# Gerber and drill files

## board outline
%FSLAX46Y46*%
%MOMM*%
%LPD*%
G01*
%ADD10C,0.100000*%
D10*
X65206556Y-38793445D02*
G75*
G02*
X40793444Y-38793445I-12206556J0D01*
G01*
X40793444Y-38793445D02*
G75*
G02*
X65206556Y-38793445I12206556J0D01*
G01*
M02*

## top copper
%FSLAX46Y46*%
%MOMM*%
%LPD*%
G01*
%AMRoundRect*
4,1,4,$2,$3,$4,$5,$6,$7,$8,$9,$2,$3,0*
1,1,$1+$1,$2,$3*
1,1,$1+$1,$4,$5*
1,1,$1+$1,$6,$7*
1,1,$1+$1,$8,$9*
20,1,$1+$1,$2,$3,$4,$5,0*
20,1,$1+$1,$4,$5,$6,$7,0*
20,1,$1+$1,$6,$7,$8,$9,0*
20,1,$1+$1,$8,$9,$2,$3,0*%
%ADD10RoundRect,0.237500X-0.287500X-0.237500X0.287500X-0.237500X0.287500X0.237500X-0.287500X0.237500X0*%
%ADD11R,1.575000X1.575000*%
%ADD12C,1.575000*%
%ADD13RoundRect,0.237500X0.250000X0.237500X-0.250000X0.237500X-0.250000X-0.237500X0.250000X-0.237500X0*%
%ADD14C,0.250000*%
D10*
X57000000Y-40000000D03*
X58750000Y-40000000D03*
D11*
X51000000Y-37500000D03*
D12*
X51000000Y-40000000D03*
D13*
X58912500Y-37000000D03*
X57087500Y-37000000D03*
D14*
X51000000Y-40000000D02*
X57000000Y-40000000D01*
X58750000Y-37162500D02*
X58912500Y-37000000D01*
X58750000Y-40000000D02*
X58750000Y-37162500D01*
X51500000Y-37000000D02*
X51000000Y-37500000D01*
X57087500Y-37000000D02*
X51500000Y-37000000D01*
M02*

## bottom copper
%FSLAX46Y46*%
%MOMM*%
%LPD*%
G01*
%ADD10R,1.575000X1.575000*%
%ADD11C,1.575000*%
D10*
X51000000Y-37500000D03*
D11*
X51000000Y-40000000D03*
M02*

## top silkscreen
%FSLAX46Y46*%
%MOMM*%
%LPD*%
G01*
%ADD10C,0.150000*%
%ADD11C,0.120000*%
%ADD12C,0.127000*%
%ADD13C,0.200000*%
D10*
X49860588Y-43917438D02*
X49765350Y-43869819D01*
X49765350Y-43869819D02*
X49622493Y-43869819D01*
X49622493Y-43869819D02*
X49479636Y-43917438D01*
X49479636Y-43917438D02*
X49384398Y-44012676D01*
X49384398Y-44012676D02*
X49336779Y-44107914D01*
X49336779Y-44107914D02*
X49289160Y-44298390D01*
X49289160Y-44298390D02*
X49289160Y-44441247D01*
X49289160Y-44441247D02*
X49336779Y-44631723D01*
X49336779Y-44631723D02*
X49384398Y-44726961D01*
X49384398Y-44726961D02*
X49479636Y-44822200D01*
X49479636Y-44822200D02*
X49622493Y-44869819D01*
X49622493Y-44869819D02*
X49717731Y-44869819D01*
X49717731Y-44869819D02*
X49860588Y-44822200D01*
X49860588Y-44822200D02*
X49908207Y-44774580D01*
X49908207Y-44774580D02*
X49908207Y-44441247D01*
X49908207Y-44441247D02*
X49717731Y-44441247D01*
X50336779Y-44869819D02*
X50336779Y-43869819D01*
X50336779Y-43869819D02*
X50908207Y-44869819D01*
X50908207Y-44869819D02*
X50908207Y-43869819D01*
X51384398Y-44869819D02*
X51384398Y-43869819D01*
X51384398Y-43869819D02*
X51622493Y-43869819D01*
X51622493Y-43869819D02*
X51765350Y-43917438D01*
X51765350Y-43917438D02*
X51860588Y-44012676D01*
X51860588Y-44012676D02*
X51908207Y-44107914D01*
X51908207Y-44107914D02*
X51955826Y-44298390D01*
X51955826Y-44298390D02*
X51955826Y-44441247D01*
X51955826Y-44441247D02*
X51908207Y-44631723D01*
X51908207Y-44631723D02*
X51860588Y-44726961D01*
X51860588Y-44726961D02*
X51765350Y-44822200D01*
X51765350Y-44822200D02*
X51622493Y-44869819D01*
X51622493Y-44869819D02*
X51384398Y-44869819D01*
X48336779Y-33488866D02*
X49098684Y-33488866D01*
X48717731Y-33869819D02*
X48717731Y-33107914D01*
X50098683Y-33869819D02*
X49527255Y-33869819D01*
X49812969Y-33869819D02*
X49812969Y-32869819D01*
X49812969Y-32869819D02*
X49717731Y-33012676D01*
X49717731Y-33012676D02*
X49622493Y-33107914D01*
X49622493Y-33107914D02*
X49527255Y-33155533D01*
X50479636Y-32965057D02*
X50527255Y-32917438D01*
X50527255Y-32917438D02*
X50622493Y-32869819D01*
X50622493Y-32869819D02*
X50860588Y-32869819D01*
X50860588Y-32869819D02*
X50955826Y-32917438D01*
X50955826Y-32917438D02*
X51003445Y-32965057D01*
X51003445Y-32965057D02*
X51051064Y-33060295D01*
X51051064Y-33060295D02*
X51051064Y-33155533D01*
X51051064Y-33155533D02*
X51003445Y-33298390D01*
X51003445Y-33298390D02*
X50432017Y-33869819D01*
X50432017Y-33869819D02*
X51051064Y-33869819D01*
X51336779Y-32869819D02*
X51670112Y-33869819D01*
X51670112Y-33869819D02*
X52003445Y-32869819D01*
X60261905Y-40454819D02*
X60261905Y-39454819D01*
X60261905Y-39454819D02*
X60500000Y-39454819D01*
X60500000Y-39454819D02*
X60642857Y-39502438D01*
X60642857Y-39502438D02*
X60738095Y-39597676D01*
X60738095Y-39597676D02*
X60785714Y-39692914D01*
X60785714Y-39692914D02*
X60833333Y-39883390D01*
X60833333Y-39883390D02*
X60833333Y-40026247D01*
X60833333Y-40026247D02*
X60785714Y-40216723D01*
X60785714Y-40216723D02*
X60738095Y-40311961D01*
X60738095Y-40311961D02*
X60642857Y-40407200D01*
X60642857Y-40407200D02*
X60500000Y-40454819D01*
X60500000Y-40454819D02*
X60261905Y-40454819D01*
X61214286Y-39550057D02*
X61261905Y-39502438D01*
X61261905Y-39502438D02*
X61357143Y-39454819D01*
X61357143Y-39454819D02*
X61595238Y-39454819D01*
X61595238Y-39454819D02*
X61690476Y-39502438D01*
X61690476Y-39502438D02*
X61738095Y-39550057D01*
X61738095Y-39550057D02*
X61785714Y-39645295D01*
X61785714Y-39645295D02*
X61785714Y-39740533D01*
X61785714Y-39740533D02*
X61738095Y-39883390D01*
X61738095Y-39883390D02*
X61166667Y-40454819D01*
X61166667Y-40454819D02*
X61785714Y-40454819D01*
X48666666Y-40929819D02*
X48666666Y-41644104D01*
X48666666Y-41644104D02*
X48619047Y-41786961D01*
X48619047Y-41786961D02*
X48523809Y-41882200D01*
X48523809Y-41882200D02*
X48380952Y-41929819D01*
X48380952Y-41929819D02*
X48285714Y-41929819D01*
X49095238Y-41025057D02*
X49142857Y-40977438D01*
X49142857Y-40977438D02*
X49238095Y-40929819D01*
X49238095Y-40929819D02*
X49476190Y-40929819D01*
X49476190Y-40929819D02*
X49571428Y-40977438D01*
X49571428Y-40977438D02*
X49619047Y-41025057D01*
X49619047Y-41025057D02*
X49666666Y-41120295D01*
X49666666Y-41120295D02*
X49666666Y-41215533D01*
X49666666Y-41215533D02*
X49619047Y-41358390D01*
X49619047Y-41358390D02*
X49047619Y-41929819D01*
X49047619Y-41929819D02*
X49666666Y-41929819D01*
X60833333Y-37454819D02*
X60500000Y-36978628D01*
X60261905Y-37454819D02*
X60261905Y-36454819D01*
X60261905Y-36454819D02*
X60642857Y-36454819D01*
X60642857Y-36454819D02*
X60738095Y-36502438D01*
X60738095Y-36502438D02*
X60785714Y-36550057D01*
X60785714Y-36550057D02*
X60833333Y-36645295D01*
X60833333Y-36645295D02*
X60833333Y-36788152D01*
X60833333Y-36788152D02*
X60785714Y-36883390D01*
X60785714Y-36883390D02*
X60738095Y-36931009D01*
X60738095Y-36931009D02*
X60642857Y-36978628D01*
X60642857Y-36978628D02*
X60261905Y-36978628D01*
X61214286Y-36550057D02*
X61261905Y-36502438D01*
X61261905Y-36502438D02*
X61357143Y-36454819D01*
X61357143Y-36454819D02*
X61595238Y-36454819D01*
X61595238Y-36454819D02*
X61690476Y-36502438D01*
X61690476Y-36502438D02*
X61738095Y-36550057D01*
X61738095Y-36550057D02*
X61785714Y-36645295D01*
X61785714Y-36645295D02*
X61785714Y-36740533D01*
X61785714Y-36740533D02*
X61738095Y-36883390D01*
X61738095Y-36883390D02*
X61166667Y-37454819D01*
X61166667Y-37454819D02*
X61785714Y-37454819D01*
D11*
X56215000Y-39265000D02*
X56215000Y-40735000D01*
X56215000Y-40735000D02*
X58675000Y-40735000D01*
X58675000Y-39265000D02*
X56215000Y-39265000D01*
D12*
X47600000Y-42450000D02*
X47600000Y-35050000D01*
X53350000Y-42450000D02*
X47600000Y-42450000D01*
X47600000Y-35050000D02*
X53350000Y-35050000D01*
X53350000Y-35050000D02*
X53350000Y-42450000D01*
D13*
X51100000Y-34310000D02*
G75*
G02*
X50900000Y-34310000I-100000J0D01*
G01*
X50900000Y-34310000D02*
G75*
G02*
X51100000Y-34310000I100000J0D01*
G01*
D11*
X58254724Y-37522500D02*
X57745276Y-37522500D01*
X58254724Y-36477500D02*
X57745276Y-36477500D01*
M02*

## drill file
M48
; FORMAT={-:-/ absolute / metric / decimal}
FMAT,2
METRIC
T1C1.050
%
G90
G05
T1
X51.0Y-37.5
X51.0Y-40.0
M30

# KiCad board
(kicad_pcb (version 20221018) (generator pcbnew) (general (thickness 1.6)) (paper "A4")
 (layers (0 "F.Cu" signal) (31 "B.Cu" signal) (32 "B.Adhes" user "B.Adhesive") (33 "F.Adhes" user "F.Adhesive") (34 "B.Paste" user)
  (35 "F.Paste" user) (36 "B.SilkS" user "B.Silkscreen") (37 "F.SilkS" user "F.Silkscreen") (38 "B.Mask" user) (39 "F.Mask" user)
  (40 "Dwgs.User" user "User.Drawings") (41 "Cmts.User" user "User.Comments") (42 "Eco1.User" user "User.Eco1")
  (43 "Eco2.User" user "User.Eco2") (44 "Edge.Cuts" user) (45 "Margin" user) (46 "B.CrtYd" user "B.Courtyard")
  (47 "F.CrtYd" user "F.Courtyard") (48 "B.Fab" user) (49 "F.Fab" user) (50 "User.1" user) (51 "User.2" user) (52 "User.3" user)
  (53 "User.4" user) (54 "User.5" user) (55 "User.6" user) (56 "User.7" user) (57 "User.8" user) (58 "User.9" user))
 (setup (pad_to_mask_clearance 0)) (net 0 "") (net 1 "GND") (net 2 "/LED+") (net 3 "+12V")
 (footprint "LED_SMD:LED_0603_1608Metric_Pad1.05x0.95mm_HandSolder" (layer "F.Cu") (at 57.875 40)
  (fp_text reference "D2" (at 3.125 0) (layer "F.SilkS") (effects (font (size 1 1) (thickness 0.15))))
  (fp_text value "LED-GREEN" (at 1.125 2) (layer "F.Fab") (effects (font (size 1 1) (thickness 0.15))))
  (fp_line (start -1.66 -0.735) (end -1.66 0.735) (stroke (width 0.12) (type solid)) (layer "F.SilkS"))
  (fp_line (start -1.66 0.735) (end 0.8 0.735) (stroke (width 0.12) (type solid)) (layer "F.SilkS"))
  (fp_line (start 0.8 -0.735) (end -1.66 -0.735) (stroke (width 0.12) (type solid)) (layer "F.SilkS"))
  (pad "1" smd roundrect (at -0.875 0) (size 1.05 0.95) (layers "F.Cu" "F.Paste" "F.Mask") (roundrect_rratio 0.25) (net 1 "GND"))
  (pad "2" smd roundrect (at 0.875 0) (size 1.05 0.95) (layers "F.Cu" "F.Paste" "F.Mask") (roundrect_rratio 0.25) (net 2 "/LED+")))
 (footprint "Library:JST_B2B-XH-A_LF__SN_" (layer "F.Cu") (at 50.475 38.75 90)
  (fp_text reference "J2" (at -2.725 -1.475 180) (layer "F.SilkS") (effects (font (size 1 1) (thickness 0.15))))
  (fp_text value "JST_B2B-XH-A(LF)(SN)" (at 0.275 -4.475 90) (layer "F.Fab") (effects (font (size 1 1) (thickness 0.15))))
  (fp_line (start -3.7 -2.875) (end 3.7 -2.875) (stroke (width 0.127) (type solid)) (layer "F.SilkS"))
  (fp_line (start -3.7 2.875) (end -3.7 -2.875) (stroke (width 0.127) (type solid)) (layer "F.SilkS"))
  (fp_line (start 3.7 -2.875) (end 3.7 2.875) (stroke (width 0.127) (type solid)) (layer "F.SilkS"))
  (fp_line (start 3.7 2.875) (end -3.7 2.875) (stroke (width 0.127) (type solid)) (layer "F.SilkS"))
  (fp_circle (center 4.44 0.525) (end 4.54 0.525) (stroke (width 0.2) (type solid)) (fill none) (layer "F.SilkS"))
  (pad "1" thru_hole rect (at 1.25 0.525 90) (size 1.575 1.575) (drill 1.05) (layers "*.Cu" "*.Mask") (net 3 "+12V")
   (solder_mask_margin 0.102))
  (pad "2" thru_hole circle (at -1.25 0.525 90) (size 1.575 1.575) (drill 1.05) (layers "*.Cu" "*.Mask") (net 1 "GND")
   (solder_mask_margin 0.102)))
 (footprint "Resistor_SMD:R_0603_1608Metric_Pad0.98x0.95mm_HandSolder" (layer "F.Cu") (at 58 37 180)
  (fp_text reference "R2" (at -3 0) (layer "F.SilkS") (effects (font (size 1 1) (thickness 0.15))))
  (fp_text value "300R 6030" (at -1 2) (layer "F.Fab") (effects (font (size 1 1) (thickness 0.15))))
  (fp_line (start -0.254724 -0.5225) (end 0.254724 -0.5225) (stroke (width 0.12) (type solid)) (layer "F.SilkS"))
  (fp_line (start -0.254724 0.5225) (end 0.254724 0.5225) (stroke (width 0.12) (type solid)) (layer "F.SilkS"))
  (pad "1" smd roundrect (at -0.9125 0 180) (size 0.975 0.95) (layers "F.Cu" "F.Paste" "F.Mask") (roundrect_rratio 0.25) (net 2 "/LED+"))
  (pad "2" smd roundrect (at 0.9125 0 180) (size 0.975 0.95) (layers "F.Cu" "F.Paste" "F.Mask") (roundrect_rratio 0.25) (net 3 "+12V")))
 (gr_circle (center 53 38.793445) (end 63 31.793445) (stroke (width 0.1) (type default)) (fill none) (layer "Edge.Cuts"))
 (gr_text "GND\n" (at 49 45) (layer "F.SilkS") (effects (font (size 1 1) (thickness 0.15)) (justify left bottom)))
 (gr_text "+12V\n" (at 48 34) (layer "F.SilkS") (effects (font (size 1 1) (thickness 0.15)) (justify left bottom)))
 (segment (start 51 40) (end 57 40) (width 0.25) (layer "F.Cu") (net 1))
 (segment (start 58.75 37.1625) (end 58.9125 37) (width 0.25) (layer "F.Cu") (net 2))
 (segment (start 58.75 40) (end 58.75 37.1625) (width 0.25) (layer "F.Cu") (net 2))
 (segment (start 51.5 37) (end 51 37.5) (width 0.25) (layer "F.Cu") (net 3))
 (segment (start 57.0875 37) (end 51.5 37) (width 0.25) (layer "F.Cu") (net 3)))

